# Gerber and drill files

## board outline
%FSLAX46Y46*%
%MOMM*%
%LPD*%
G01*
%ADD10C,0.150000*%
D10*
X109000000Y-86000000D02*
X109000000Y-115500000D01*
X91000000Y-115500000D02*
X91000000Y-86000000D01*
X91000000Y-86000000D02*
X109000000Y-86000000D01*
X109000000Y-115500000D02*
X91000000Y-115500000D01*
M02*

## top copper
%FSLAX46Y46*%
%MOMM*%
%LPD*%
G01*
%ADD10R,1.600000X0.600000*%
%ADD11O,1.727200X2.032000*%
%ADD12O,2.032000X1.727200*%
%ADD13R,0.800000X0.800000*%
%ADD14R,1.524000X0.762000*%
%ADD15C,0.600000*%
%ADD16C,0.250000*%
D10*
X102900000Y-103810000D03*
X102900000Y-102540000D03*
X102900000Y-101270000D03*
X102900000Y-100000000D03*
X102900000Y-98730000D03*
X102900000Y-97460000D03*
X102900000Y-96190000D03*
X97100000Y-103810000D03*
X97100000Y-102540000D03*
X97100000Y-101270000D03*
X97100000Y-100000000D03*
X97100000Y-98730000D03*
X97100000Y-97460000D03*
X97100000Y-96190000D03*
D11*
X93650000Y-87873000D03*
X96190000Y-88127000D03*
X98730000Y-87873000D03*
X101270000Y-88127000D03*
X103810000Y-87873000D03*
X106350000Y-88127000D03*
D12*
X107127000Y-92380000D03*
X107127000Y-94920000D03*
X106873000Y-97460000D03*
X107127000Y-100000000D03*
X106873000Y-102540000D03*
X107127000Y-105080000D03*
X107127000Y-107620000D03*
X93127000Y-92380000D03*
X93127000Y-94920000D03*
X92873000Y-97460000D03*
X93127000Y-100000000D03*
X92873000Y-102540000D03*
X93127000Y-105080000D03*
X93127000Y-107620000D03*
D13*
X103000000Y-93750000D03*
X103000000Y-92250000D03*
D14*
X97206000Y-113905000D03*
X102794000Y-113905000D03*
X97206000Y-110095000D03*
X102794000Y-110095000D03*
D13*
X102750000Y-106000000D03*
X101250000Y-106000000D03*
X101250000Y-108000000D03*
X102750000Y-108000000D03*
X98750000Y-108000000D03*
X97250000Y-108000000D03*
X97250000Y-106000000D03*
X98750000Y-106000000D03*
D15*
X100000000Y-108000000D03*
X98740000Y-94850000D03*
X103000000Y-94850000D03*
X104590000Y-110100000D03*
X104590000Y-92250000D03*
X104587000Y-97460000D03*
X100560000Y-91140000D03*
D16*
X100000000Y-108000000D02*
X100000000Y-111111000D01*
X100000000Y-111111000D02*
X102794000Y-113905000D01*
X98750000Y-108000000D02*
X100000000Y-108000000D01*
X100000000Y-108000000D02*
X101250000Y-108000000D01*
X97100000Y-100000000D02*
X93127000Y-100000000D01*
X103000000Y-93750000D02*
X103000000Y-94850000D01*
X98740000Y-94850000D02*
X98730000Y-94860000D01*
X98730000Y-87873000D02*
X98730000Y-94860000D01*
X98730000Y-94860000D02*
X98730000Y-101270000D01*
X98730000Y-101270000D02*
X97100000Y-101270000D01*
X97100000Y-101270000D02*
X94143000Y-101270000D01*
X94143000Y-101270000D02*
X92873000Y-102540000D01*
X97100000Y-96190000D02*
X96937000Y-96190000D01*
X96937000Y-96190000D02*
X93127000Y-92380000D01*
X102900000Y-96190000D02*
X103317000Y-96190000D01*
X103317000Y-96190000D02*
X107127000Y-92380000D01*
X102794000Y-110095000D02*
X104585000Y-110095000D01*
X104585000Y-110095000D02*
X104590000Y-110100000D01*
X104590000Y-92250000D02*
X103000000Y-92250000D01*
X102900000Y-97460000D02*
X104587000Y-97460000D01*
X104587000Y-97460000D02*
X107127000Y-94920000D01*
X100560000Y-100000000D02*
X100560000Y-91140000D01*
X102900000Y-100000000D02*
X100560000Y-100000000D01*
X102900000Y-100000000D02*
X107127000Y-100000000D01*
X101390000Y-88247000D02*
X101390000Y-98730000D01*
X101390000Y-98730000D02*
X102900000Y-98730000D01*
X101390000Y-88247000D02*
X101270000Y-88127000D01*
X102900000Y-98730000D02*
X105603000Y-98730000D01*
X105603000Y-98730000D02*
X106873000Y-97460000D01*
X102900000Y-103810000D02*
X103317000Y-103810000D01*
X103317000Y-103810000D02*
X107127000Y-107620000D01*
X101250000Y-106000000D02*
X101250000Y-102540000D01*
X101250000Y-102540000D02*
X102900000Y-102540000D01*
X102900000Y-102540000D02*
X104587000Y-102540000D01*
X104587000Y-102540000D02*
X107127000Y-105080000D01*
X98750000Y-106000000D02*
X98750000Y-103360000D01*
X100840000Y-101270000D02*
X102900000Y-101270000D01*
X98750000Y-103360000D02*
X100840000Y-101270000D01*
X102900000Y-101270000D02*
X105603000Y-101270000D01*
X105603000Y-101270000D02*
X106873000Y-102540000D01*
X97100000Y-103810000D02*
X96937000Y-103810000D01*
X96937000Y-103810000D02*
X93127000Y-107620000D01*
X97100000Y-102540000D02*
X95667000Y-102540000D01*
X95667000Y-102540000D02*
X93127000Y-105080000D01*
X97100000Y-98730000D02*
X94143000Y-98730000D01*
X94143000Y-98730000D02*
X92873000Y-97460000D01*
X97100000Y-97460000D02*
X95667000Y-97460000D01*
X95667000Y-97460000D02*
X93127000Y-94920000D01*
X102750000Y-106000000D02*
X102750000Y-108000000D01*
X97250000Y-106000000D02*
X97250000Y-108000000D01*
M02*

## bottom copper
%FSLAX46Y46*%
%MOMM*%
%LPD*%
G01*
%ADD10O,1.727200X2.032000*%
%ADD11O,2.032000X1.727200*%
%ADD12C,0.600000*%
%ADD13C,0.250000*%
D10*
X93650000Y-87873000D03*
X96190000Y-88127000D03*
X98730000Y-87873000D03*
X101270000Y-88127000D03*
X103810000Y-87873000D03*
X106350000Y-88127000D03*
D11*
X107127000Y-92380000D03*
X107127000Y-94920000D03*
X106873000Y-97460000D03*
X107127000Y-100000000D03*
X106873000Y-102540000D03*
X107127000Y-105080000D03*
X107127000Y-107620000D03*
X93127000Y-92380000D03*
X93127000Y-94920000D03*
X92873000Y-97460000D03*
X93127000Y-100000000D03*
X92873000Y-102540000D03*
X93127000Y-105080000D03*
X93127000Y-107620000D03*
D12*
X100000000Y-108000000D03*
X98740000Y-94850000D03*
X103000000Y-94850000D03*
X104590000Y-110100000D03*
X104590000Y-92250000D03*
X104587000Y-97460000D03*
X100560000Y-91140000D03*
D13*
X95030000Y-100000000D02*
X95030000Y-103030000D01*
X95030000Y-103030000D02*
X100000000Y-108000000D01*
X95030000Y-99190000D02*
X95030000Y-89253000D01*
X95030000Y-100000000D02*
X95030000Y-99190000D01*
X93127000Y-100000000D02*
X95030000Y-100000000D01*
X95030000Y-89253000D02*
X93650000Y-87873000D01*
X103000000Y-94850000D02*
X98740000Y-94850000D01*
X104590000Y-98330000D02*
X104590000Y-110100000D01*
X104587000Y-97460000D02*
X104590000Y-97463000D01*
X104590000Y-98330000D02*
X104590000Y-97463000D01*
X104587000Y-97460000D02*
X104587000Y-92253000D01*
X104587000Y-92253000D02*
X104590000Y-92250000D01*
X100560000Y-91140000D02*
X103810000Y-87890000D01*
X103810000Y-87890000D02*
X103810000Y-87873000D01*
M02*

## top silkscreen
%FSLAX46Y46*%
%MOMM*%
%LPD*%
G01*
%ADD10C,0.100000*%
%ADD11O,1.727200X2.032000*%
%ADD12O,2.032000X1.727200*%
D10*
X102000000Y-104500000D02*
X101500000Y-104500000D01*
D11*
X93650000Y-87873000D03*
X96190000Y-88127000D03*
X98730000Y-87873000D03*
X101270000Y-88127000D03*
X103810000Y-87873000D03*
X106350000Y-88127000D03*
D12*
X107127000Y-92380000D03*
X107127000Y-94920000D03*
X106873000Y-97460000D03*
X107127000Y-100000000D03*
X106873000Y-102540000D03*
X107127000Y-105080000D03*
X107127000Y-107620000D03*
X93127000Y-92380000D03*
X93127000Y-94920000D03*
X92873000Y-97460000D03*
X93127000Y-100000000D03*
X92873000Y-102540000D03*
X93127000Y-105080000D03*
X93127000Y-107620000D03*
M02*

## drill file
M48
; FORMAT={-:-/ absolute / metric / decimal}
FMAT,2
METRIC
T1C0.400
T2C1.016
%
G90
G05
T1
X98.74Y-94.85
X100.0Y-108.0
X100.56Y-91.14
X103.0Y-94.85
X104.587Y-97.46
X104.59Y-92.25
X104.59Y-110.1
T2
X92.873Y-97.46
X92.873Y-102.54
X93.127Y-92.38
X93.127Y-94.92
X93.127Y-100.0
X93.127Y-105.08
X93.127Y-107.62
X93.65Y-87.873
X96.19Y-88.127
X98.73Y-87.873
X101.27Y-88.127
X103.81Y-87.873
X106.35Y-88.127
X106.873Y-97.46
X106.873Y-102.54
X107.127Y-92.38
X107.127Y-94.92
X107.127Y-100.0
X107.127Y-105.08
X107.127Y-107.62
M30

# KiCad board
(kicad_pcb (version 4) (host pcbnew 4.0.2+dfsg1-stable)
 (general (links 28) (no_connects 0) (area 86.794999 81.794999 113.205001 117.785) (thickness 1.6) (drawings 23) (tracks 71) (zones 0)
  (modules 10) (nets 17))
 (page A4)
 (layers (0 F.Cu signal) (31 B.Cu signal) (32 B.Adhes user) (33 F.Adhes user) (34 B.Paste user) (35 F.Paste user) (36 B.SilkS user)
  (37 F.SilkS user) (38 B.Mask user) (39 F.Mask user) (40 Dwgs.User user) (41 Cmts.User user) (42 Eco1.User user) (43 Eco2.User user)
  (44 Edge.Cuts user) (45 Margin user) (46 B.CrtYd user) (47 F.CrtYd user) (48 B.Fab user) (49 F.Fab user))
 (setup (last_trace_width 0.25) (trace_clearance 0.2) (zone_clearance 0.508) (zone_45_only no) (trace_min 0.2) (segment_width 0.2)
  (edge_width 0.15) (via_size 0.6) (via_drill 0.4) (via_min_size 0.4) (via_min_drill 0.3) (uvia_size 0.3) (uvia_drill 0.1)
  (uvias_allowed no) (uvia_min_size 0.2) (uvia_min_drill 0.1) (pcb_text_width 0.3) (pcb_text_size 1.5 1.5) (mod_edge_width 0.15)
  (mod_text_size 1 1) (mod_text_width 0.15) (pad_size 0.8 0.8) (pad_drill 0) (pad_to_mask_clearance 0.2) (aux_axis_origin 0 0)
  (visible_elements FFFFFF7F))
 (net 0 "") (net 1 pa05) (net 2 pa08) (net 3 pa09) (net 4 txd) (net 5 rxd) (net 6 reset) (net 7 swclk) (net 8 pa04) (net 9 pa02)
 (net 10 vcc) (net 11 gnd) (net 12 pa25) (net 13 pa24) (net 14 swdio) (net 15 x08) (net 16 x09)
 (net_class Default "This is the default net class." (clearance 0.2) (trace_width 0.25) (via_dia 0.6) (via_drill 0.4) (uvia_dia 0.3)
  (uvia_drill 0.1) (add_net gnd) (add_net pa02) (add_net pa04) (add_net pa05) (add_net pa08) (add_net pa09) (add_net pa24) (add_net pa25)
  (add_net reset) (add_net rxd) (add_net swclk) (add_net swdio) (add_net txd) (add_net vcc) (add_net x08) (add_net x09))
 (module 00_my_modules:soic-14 (layer F.Cu) (at 100 100 180)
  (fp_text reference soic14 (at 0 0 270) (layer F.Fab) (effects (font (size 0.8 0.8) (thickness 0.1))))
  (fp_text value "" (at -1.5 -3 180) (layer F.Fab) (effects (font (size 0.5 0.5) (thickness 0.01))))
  (fp_line (start -2 -4.5) (end -1.5 -4.5) (layer F.SilkS) (width 0.1))
  (pad PA05 smd rect (at -2.9 -3.81 180) (size 1.6 0.6) (layers F.Cu F.Paste F.Mask) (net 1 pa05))
  (pad PA08 smd rect (at -2.9 -2.54 180) (size 1.6 0.6) (layers F.Cu F.Paste F.Mask) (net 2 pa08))
  (pad PA09 smd rect (at -2.9 -1.27 180) (size 1.6 0.6) (layers F.Cu F.Paste F.Mask) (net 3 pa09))
  (pad PA14 smd rect (at -2.9 0 180) (size 1.6 0.6) (layers F.Cu F.Paste F.Mask) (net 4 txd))
  (pad PA15 smd rect (at -2.9 1.27 180) (size 1.6 0.6) (layers F.Cu F.Paste F.Mask) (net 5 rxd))
  (pad RST smd rect (at -2.9 2.54 180) (size 1.6 0.6) (layers F.Cu F.Paste F.Mask) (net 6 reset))
  (pad PA30 smd rect (at -2.9 3.81 180) (size 1.6 0.6) (layers F.Cu F.Paste F.Mask) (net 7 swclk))
  (pad PA04 smd rect (at 2.9 -3.81 180) (size 1.6 0.6) (layers F.Cu F.Paste F.Mask) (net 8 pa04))
  (pad PA02 smd rect (at 2.9 -2.54 180) (size 1.6 0.6) (layers F.Cu F.Paste F.Mask) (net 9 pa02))
  (pad VDD smd rect (at 2.9 -1.27 180) (size 1.6 0.6) (layers F.Cu F.Paste F.Mask) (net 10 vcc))
  (pad GND smd rect (at 2.9 0 180) (size 1.6 0.6) (layers F.Cu F.Paste F.Mask) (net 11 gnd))
  (pad PA25 smd rect (at 2.9 1.27 180) (size 1.6 0.6) (layers F.Cu F.Paste F.Mask) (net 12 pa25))
  (pad PA24 smd rect (at 2.9 2.54 180) (size 1.6 0.6) (layers F.Cu F.Paste F.Mask) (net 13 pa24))
  (pad PA31 smd rect (at 2.9 3.81 180) (size 1.6 0.6) (layers F.Cu F.Paste F.Mask) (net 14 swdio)))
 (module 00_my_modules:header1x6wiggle (layer F.Cu) (at 100 88 90)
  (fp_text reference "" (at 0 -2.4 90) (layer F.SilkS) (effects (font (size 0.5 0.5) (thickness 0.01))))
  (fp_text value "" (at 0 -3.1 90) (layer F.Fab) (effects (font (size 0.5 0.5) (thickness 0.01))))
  (pad GND thru_hole oval (at 0.127 -6.35 90) (size 2.032 1.7272) (drill 1.016) (layers *.Cu *.Mask F.SilkS) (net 11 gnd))
  (pad 2 thru_hole oval (at -0.127 -3.81 90) (size 2.032 1.7272) (drill 1.016) (layers *.Cu *.Mask F.SilkS))
  (pad VCC thru_hole oval (at 0.127 -1.27 90) (size 2.032 1.7272) (drill 1.016) (layers *.Cu *.Mask F.SilkS) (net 10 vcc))
  (pad TX thru_hole oval (at -0.127 1.27 90) (size 2.032 1.7272) (drill 1.016) (layers *.Cu *.Mask F.SilkS) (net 5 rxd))
  (pad RX thru_hole oval (at 0.127 3.81 90) (size 2.032 1.7272) (drill 1.016) (layers *.Cu *.Mask F.SilkS) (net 4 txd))
  (pad 6 thru_hole oval (at -0.127 6.35 90) (size 2.032 1.7272) (drill 1.016) (layers *.Cu *.Mask F.SilkS)))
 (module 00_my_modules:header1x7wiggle (layer F.Cu) (at 107 100)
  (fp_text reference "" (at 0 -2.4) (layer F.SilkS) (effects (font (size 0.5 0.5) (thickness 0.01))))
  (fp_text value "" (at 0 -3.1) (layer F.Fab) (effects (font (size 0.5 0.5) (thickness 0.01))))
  (pad 1 thru_hole oval (at 0.127 -7.62) (size 2.032 1.7272) (drill 1.016) (layers *.Cu *.Mask F.SilkS) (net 7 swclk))
  (pad 2 thru_hole oval (at 0.127 -5.08) (size 2.032 1.7272) (drill 1.016) (layers *.Cu *.Mask F.SilkS) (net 6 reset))
  (pad 3 thru_hole oval (at -0.127 -2.54) (size 2.032 1.7272) (drill 1.016) (layers *.Cu *.Mask F.SilkS) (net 5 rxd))
  (pad 4 thru_hole oval (at 0.127 0) (size 2.032 1.7272) (drill 1.016) (layers *.Cu *.Mask F.SilkS) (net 4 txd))
  (pad 5 thru_hole oval (at -0.127 2.54) (size 2.032 1.7272) (drill 1.016) (layers *.Cu *.Mask F.SilkS) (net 3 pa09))
  (pad 6 thru_hole oval (at 0.127 5.08) (size 2.032 1.7272) (drill 1.016) (layers *.Cu *.Mask F.SilkS) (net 2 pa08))
  (pad 7 thru_hole oval (at 0.127 7.62) (size 2.032 1.7272) (drill 1.016) (layers *.Cu *.Mask F.SilkS) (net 1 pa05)))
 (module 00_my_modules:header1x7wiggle (layer F.Cu) (at 93 100)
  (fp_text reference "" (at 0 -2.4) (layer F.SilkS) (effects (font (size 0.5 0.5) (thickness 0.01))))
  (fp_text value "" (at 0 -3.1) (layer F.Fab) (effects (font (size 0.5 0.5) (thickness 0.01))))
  (pad 1 thru_hole oval (at 0.127 -7.62) (size 2.032 1.7272) (drill 1.016) (layers *.Cu *.Mask F.SilkS) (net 14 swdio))
  (pad 2 thru_hole oval (at 0.127 -5.08) (size 2.032 1.7272) (drill 1.016) (layers *.Cu *.Mask F.SilkS) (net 13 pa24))
  (pad 3 thru_hole oval (at -0.127 -2.54) (size 2.032 1.7272) (drill 1.016) (layers *.Cu *.Mask F.SilkS) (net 12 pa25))
  (pad 4 thru_hole oval (at 0.127 0) (size 2.032 1.7272) (drill 1.016) (layers *.Cu *.Mask F.SilkS) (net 11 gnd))
  (pad 5 thru_hole oval (at -0.127 2.54) (size 2.032 1.7272) (drill 1.016) (layers *.Cu *.Mask F.SilkS) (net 10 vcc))
  (pad 6 thru_hole oval (at 0.127 5.08) (size 2.032 1.7272) (drill 1.016) (layers *.Cu *.Mask F.SilkS) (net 9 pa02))
  (pad 7 thru_hole oval (at 0.127 7.62) (size 2.032 1.7272) (drill 1.016) (layers *.Cu *.Mask F.SilkS) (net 8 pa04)))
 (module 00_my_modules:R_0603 (layer F.Cu) (at 103 93 90)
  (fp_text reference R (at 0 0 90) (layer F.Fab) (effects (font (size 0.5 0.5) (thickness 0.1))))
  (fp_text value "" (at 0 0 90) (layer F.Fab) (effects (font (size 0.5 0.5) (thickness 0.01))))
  (pad 1 smd rect (at -0.75 0 90) (size 0.8 0.8) (layers F.Cu F.Paste F.Mask) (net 10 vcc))
  (pad 2 smd rect (at 0.75 0 90) (size 0.8 0.8) (layers F.Cu F.Paste F.Mask) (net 6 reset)))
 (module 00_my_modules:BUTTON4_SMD (layer F.Cu) (at 100 112)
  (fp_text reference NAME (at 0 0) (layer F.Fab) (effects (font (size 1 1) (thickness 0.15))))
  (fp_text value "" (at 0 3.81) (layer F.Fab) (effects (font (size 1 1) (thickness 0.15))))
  (pad 1 smd rect (at -2.794 1.905) (size 1.524 0.762) (layers F.Cu F.Paste F.Mask))
  (pad 2 smd rect (at 2.794 1.905) (size 1.524 0.762) (layers F.Cu F.Paste F.Mask) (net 11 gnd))
  (pad 3 smd rect (at -2.794 -1.905) (size 1.524 0.762) (layers F.Cu F.Paste F.Mask))
  (pad 4 smd rect (at 2.794 -1.905) (size 1.524 0.762) (layers F.Cu F.Paste F.Mask) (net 6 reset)))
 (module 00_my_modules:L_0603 (layer F.Cu) (at 102 106 180)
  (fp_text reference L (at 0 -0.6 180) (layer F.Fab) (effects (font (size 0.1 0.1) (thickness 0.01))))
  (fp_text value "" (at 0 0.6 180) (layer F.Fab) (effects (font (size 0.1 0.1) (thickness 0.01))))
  (pad 1 smd rect (at -0.75 0 180) (size 0.8 0.8) (layers F.Cu F.Paste F.Mask) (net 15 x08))
  (pad 2 smd rect (at 0.75 0 180) (size 0.8 0.8) (layers F.Cu F.Paste F.Mask) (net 2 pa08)))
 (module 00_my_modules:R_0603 (layer F.Cu) (at 102 108)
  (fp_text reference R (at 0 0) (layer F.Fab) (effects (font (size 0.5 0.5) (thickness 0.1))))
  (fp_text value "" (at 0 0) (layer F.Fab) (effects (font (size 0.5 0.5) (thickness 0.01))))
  (pad 1 smd rect (at -0.75 0) (size 0.8 0.8) (layers F.Cu F.Paste F.Mask) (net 11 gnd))
  (pad 2 smd rect (at 0.75 0) (size 0.8 0.8) (layers F.Cu F.Paste F.Mask) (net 15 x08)))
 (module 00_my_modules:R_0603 (layer F.Cu) (at 98 108 180)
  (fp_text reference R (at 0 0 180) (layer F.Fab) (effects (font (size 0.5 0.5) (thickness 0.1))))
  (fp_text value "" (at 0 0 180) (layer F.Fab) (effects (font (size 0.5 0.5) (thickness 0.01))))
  (pad 1 smd rect (at -0.75 0 180) (size 0.8 0.8) (layers F.Cu F.Paste F.Mask) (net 11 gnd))
  (pad 2 smd rect (at 0.75 0 180) (size 0.8 0.8) (layers F.Cu F.Paste F.Mask) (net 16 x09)))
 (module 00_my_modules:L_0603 (layer F.Cu) (at 98 106)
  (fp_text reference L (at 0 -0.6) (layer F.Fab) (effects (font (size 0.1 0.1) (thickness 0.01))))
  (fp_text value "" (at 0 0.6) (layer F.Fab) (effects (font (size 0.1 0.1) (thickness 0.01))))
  (pad 1 smd rect (at -0.75 0) (size 0.8 0.8) (layers F.Cu F.Paste F.Mask) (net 16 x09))
  (pad 2 smd rect (at 0.75 0) (size 0.8 0.8) (layers F.Cu F.Paste F.Mask) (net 3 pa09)))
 (gr_line (start 109 86) (end 109 115.5) (angle 90) (layer Edge.Cuts) (width 0.15))
 (gr_line (start 91 115.5) (end 91 86) (angle 90) (layer Edge.Cuts) (width 0.15))
 (gr_line (start 91 86) (end 109 86) (angle 90) (layer Edge.Cuts) (width 0.15))
 (gr_line (start 109 115.5) (end 91 115.5) (angle 90) (layer Edge.Cuts) (width 0.15))
 (segment (start 100 108) (end 100 111.111) (width 0.25) (layer F.Cu) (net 11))
 (segment (start 100 111.111) (end 102.794 113.905) (width 0.25) (layer F.Cu) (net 11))
 (segment (start 95.03 100) (end 95.03 103.03) (width 0.25) (layer B.Cu) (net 11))
 (via (at 100 108) (size 0.6) (drill 0.4) (layers F.Cu B.Cu) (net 11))
 (segment (start 95.03 103.03) (end 100 108) (width 0.25) (layer B.Cu) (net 11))
 (segment (start 98.75 108) (end 100 108) (width 0.25) (layer F.Cu) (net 11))
 (segment (start 100 108) (end 101.25 108) (width 0.25) (layer F.Cu) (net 11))
 (segment (start 95.03 99.19) (end 95.03 89.253) (width 0.25) (layer B.Cu) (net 11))
 (segment (start 95.03 100) (end 95.03 99.19) (width 0.25) (layer B.Cu) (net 11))
 (segment (start 93.127 100) (end 95.03 100) (width 0.25) (layer B.Cu) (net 11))
 (segment (start 95.03 89.253) (end 93.65 87.873) (width 0.25) (layer B.Cu) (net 11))
 (segment (start 97.1 100) (end 93.127 100) (width 0.25) (layer F.Cu) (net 11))
 (segment (start 103 93.75) (end 103 94.85) (width 0.25) (layer F.Cu) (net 10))
 (segment (start 98.74 94.85) (end 98.73 94.86) (width 0.25) (layer F.Cu) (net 10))
 (via (at 98.74 94.85) (size 0.6) (drill 0.4) (layers F.Cu B.Cu) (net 10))
 (segment (start 103 94.85) (end 98.74 94.85) (width 0.25) (layer B.Cu) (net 10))
 (via (at 103 94.85) (size 0.6) (drill 0.4) (layers F.Cu B.Cu) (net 10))
 (segment (start 98.73 87.873) (end 98.73 94.86) (width 0.25) (layer F.Cu) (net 10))
 (segment (start 98.73 94.86) (end 98.73 101.27) (width 0.25) (layer F.Cu) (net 10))
 (segment (start 98.73 101.27) (end 97.1 101.27) (width 0.25) (layer F.Cu) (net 10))
 (segment (start 97.1 101.27) (end 94.143 101.27) (width 0.25) (layer F.Cu) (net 10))
 (segment (start 94.143 101.27) (end 92.873 102.54) (width 0.25) (layer F.Cu) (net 10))
 (segment (start 97.1 96.19) (end 96.937 96.19) (width 0.25) (layer F.Cu) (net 14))
 (segment (start 96.937 96.19) (end 93.127 92.38) (width 0.25) (layer F.Cu) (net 14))
 (segment (start 102.9 96.19) (end 103.317 96.19) (width 0.25) (layer F.Cu) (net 7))
 (segment (start 103.317 96.19) (end 107.127 92.38) (width 0.25) (layer F.Cu) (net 7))
 (segment (start 102.794 110.095) (end 104.585 110.095) (width 0.25) (layer F.Cu) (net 6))
 (via (at 104.59 110.1) (size 0.6) (drill 0.4) (layers F.Cu B.Cu) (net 6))
 (segment (start 104.585 110.095) (end 104.59 110.1) (width 0.25) (layer F.Cu) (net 6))
 (segment (start 104.59 98.33) (end 104.59 110.1) (width 0.25) (layer B.Cu) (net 6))
 (segment (start 104.587 97.46) (end 104.59 97.463) (width 0.25) (layer B.Cu) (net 6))
 (segment (start 104.59 98.33) (end 104.59 97.463) (width 0.25) (layer B.Cu) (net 6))
 (segment (start 104.587 97.46) (end 104.587 92.253) (width 0.25) (layer B.Cu) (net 6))
 (segment (start 104.59 92.25) (end 103 92.25) (width 0.25) (layer F.Cu) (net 6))
 (via (at 104.59 92.25) (size 0.6) (drill 0.4) (layers F.Cu B.Cu) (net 6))
 (segment (start 104.587 92.253) (end 104.59 92.25) (width 0.25) (layer B.Cu) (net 6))
 (via (at 104.587 97.46) (size 0.6) (drill 0.4) (layers F.Cu B.Cu) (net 6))
 (segment (start 102.9 97.46) (end 104.587 97.46) (width 0.25) (layer F.Cu) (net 6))
 (segment (start 104.587 97.46) (end 107.127 94.92) (width 0.25) (layer F.Cu) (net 6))
 (segment (start 100.56 100) (end 100.56 91.14) (width 0.25) (layer F.Cu) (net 4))
 (segment (start 102.9 100) (end 100.56 100) (width 0.25) (layer F.Cu) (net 4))
 (segment (start 100.56 91.14) (end 103.81 87.89) (width 0.25) (layer B.Cu) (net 4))
 (via (at 100.56 91.14) (size 0.6) (drill 0.4) (layers F.Cu B.Cu) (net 4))
 (segment (start 103.81 87.89) (end 103.81 87.873) (width 0.25) (layer B.Cu) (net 4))
 (segment (start 102.9 100) (end 107.127 100) (width 0.25) (layer F.Cu) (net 4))
 (segment (start 101.39 88.247) (end 101.39 98.73) (width 0.25) (layer F.Cu) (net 5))
 (segment (start 101.39 98.73) (end 102.9 98.73) (width 0.25) (layer F.Cu) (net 5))
 (segment (start 101.39 88.247) (end 101.27 88.127) (width 0.25) (layer F.Cu) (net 5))
 (segment (start 102.9 98.73) (end 105.603 98.73) (width 0.25) (layer F.Cu) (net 5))
 (segment (start 105.603 98.73) (end 106.873 97.46) (width 0.25) (layer F.Cu) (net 5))
 (segment (start 102.9 103.81) (end 103.317 103.81) (width 0.25) (layer F.Cu) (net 1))
 (segment (start 103.317 103.81) (end 107.127 107.62) (width 0.25) (layer F.Cu) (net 1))
 (segment (start 101.25 106) (end 101.25 102.54) (width 0.25) (layer F.Cu) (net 2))
 (segment (start 101.25 102.54) (end 102.9 102.54) (width 0.25) (layer F.Cu) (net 2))
 (segment (start 102.9 102.54) (end 104.587 102.54) (width 0.25) (layer F.Cu) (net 2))
 (segment (start 104.587 102.54) (end 107.127 105.08) (width 0.25) (layer F.Cu) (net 2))
 (segment (start 98.75 106) (end 98.75 103.36) (width 0.25) (layer F.Cu) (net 3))
 (segment (start 100.84 101.27) (end 102.9 101.27) (width 0.25) (layer F.Cu) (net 3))
 (segment (start 98.75 103.36) (end 100.84 101.27) (width 0.25) (layer F.Cu) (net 3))
 (segment (start 102.9 101.27) (end 105.603 101.27) (width 0.25) (layer F.Cu) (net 3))
 (segment (start 105.603 101.27) (end 106.873 102.54) (width 0.25) (layer F.Cu) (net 3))
 (segment (start 97.1 103.81) (end 96.937 103.81) (width 0.25) (layer F.Cu) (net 8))
 (segment (start 96.937 103.81) (end 93.127 107.62) (width 0.25) (layer F.Cu) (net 8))
 (segment (start 97.1 102.54) (end 95.667 102.54) (width 0.25) (layer F.Cu) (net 9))
 (segment (start 95.667 102.54) (end 93.127 105.08) (width 0.25) (layer F.Cu) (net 9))
 (segment (start 97.1 98.73) (end 94.143 98.73) (width 0.25) (layer F.Cu) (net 12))
 (segment (start 94.143 98.73) (end 92.873 97.46) (width 0.25) (layer F.Cu) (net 12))
 (segment (start 97.1 97.46) (end 95.667 97.46) (width 0.25) (layer F.Cu) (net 13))
 (segment (start 95.667 97.46) (end 93.127 94.92) (width 0.25) (layer F.Cu) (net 13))
 (segment (start 102.75 106) (end 102.75 108) (width 0.25) (layer F.Cu) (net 15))
 (segment (start 97.25 106) (end 97.25 108) (width 0.25) (layer F.Cu) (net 16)))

